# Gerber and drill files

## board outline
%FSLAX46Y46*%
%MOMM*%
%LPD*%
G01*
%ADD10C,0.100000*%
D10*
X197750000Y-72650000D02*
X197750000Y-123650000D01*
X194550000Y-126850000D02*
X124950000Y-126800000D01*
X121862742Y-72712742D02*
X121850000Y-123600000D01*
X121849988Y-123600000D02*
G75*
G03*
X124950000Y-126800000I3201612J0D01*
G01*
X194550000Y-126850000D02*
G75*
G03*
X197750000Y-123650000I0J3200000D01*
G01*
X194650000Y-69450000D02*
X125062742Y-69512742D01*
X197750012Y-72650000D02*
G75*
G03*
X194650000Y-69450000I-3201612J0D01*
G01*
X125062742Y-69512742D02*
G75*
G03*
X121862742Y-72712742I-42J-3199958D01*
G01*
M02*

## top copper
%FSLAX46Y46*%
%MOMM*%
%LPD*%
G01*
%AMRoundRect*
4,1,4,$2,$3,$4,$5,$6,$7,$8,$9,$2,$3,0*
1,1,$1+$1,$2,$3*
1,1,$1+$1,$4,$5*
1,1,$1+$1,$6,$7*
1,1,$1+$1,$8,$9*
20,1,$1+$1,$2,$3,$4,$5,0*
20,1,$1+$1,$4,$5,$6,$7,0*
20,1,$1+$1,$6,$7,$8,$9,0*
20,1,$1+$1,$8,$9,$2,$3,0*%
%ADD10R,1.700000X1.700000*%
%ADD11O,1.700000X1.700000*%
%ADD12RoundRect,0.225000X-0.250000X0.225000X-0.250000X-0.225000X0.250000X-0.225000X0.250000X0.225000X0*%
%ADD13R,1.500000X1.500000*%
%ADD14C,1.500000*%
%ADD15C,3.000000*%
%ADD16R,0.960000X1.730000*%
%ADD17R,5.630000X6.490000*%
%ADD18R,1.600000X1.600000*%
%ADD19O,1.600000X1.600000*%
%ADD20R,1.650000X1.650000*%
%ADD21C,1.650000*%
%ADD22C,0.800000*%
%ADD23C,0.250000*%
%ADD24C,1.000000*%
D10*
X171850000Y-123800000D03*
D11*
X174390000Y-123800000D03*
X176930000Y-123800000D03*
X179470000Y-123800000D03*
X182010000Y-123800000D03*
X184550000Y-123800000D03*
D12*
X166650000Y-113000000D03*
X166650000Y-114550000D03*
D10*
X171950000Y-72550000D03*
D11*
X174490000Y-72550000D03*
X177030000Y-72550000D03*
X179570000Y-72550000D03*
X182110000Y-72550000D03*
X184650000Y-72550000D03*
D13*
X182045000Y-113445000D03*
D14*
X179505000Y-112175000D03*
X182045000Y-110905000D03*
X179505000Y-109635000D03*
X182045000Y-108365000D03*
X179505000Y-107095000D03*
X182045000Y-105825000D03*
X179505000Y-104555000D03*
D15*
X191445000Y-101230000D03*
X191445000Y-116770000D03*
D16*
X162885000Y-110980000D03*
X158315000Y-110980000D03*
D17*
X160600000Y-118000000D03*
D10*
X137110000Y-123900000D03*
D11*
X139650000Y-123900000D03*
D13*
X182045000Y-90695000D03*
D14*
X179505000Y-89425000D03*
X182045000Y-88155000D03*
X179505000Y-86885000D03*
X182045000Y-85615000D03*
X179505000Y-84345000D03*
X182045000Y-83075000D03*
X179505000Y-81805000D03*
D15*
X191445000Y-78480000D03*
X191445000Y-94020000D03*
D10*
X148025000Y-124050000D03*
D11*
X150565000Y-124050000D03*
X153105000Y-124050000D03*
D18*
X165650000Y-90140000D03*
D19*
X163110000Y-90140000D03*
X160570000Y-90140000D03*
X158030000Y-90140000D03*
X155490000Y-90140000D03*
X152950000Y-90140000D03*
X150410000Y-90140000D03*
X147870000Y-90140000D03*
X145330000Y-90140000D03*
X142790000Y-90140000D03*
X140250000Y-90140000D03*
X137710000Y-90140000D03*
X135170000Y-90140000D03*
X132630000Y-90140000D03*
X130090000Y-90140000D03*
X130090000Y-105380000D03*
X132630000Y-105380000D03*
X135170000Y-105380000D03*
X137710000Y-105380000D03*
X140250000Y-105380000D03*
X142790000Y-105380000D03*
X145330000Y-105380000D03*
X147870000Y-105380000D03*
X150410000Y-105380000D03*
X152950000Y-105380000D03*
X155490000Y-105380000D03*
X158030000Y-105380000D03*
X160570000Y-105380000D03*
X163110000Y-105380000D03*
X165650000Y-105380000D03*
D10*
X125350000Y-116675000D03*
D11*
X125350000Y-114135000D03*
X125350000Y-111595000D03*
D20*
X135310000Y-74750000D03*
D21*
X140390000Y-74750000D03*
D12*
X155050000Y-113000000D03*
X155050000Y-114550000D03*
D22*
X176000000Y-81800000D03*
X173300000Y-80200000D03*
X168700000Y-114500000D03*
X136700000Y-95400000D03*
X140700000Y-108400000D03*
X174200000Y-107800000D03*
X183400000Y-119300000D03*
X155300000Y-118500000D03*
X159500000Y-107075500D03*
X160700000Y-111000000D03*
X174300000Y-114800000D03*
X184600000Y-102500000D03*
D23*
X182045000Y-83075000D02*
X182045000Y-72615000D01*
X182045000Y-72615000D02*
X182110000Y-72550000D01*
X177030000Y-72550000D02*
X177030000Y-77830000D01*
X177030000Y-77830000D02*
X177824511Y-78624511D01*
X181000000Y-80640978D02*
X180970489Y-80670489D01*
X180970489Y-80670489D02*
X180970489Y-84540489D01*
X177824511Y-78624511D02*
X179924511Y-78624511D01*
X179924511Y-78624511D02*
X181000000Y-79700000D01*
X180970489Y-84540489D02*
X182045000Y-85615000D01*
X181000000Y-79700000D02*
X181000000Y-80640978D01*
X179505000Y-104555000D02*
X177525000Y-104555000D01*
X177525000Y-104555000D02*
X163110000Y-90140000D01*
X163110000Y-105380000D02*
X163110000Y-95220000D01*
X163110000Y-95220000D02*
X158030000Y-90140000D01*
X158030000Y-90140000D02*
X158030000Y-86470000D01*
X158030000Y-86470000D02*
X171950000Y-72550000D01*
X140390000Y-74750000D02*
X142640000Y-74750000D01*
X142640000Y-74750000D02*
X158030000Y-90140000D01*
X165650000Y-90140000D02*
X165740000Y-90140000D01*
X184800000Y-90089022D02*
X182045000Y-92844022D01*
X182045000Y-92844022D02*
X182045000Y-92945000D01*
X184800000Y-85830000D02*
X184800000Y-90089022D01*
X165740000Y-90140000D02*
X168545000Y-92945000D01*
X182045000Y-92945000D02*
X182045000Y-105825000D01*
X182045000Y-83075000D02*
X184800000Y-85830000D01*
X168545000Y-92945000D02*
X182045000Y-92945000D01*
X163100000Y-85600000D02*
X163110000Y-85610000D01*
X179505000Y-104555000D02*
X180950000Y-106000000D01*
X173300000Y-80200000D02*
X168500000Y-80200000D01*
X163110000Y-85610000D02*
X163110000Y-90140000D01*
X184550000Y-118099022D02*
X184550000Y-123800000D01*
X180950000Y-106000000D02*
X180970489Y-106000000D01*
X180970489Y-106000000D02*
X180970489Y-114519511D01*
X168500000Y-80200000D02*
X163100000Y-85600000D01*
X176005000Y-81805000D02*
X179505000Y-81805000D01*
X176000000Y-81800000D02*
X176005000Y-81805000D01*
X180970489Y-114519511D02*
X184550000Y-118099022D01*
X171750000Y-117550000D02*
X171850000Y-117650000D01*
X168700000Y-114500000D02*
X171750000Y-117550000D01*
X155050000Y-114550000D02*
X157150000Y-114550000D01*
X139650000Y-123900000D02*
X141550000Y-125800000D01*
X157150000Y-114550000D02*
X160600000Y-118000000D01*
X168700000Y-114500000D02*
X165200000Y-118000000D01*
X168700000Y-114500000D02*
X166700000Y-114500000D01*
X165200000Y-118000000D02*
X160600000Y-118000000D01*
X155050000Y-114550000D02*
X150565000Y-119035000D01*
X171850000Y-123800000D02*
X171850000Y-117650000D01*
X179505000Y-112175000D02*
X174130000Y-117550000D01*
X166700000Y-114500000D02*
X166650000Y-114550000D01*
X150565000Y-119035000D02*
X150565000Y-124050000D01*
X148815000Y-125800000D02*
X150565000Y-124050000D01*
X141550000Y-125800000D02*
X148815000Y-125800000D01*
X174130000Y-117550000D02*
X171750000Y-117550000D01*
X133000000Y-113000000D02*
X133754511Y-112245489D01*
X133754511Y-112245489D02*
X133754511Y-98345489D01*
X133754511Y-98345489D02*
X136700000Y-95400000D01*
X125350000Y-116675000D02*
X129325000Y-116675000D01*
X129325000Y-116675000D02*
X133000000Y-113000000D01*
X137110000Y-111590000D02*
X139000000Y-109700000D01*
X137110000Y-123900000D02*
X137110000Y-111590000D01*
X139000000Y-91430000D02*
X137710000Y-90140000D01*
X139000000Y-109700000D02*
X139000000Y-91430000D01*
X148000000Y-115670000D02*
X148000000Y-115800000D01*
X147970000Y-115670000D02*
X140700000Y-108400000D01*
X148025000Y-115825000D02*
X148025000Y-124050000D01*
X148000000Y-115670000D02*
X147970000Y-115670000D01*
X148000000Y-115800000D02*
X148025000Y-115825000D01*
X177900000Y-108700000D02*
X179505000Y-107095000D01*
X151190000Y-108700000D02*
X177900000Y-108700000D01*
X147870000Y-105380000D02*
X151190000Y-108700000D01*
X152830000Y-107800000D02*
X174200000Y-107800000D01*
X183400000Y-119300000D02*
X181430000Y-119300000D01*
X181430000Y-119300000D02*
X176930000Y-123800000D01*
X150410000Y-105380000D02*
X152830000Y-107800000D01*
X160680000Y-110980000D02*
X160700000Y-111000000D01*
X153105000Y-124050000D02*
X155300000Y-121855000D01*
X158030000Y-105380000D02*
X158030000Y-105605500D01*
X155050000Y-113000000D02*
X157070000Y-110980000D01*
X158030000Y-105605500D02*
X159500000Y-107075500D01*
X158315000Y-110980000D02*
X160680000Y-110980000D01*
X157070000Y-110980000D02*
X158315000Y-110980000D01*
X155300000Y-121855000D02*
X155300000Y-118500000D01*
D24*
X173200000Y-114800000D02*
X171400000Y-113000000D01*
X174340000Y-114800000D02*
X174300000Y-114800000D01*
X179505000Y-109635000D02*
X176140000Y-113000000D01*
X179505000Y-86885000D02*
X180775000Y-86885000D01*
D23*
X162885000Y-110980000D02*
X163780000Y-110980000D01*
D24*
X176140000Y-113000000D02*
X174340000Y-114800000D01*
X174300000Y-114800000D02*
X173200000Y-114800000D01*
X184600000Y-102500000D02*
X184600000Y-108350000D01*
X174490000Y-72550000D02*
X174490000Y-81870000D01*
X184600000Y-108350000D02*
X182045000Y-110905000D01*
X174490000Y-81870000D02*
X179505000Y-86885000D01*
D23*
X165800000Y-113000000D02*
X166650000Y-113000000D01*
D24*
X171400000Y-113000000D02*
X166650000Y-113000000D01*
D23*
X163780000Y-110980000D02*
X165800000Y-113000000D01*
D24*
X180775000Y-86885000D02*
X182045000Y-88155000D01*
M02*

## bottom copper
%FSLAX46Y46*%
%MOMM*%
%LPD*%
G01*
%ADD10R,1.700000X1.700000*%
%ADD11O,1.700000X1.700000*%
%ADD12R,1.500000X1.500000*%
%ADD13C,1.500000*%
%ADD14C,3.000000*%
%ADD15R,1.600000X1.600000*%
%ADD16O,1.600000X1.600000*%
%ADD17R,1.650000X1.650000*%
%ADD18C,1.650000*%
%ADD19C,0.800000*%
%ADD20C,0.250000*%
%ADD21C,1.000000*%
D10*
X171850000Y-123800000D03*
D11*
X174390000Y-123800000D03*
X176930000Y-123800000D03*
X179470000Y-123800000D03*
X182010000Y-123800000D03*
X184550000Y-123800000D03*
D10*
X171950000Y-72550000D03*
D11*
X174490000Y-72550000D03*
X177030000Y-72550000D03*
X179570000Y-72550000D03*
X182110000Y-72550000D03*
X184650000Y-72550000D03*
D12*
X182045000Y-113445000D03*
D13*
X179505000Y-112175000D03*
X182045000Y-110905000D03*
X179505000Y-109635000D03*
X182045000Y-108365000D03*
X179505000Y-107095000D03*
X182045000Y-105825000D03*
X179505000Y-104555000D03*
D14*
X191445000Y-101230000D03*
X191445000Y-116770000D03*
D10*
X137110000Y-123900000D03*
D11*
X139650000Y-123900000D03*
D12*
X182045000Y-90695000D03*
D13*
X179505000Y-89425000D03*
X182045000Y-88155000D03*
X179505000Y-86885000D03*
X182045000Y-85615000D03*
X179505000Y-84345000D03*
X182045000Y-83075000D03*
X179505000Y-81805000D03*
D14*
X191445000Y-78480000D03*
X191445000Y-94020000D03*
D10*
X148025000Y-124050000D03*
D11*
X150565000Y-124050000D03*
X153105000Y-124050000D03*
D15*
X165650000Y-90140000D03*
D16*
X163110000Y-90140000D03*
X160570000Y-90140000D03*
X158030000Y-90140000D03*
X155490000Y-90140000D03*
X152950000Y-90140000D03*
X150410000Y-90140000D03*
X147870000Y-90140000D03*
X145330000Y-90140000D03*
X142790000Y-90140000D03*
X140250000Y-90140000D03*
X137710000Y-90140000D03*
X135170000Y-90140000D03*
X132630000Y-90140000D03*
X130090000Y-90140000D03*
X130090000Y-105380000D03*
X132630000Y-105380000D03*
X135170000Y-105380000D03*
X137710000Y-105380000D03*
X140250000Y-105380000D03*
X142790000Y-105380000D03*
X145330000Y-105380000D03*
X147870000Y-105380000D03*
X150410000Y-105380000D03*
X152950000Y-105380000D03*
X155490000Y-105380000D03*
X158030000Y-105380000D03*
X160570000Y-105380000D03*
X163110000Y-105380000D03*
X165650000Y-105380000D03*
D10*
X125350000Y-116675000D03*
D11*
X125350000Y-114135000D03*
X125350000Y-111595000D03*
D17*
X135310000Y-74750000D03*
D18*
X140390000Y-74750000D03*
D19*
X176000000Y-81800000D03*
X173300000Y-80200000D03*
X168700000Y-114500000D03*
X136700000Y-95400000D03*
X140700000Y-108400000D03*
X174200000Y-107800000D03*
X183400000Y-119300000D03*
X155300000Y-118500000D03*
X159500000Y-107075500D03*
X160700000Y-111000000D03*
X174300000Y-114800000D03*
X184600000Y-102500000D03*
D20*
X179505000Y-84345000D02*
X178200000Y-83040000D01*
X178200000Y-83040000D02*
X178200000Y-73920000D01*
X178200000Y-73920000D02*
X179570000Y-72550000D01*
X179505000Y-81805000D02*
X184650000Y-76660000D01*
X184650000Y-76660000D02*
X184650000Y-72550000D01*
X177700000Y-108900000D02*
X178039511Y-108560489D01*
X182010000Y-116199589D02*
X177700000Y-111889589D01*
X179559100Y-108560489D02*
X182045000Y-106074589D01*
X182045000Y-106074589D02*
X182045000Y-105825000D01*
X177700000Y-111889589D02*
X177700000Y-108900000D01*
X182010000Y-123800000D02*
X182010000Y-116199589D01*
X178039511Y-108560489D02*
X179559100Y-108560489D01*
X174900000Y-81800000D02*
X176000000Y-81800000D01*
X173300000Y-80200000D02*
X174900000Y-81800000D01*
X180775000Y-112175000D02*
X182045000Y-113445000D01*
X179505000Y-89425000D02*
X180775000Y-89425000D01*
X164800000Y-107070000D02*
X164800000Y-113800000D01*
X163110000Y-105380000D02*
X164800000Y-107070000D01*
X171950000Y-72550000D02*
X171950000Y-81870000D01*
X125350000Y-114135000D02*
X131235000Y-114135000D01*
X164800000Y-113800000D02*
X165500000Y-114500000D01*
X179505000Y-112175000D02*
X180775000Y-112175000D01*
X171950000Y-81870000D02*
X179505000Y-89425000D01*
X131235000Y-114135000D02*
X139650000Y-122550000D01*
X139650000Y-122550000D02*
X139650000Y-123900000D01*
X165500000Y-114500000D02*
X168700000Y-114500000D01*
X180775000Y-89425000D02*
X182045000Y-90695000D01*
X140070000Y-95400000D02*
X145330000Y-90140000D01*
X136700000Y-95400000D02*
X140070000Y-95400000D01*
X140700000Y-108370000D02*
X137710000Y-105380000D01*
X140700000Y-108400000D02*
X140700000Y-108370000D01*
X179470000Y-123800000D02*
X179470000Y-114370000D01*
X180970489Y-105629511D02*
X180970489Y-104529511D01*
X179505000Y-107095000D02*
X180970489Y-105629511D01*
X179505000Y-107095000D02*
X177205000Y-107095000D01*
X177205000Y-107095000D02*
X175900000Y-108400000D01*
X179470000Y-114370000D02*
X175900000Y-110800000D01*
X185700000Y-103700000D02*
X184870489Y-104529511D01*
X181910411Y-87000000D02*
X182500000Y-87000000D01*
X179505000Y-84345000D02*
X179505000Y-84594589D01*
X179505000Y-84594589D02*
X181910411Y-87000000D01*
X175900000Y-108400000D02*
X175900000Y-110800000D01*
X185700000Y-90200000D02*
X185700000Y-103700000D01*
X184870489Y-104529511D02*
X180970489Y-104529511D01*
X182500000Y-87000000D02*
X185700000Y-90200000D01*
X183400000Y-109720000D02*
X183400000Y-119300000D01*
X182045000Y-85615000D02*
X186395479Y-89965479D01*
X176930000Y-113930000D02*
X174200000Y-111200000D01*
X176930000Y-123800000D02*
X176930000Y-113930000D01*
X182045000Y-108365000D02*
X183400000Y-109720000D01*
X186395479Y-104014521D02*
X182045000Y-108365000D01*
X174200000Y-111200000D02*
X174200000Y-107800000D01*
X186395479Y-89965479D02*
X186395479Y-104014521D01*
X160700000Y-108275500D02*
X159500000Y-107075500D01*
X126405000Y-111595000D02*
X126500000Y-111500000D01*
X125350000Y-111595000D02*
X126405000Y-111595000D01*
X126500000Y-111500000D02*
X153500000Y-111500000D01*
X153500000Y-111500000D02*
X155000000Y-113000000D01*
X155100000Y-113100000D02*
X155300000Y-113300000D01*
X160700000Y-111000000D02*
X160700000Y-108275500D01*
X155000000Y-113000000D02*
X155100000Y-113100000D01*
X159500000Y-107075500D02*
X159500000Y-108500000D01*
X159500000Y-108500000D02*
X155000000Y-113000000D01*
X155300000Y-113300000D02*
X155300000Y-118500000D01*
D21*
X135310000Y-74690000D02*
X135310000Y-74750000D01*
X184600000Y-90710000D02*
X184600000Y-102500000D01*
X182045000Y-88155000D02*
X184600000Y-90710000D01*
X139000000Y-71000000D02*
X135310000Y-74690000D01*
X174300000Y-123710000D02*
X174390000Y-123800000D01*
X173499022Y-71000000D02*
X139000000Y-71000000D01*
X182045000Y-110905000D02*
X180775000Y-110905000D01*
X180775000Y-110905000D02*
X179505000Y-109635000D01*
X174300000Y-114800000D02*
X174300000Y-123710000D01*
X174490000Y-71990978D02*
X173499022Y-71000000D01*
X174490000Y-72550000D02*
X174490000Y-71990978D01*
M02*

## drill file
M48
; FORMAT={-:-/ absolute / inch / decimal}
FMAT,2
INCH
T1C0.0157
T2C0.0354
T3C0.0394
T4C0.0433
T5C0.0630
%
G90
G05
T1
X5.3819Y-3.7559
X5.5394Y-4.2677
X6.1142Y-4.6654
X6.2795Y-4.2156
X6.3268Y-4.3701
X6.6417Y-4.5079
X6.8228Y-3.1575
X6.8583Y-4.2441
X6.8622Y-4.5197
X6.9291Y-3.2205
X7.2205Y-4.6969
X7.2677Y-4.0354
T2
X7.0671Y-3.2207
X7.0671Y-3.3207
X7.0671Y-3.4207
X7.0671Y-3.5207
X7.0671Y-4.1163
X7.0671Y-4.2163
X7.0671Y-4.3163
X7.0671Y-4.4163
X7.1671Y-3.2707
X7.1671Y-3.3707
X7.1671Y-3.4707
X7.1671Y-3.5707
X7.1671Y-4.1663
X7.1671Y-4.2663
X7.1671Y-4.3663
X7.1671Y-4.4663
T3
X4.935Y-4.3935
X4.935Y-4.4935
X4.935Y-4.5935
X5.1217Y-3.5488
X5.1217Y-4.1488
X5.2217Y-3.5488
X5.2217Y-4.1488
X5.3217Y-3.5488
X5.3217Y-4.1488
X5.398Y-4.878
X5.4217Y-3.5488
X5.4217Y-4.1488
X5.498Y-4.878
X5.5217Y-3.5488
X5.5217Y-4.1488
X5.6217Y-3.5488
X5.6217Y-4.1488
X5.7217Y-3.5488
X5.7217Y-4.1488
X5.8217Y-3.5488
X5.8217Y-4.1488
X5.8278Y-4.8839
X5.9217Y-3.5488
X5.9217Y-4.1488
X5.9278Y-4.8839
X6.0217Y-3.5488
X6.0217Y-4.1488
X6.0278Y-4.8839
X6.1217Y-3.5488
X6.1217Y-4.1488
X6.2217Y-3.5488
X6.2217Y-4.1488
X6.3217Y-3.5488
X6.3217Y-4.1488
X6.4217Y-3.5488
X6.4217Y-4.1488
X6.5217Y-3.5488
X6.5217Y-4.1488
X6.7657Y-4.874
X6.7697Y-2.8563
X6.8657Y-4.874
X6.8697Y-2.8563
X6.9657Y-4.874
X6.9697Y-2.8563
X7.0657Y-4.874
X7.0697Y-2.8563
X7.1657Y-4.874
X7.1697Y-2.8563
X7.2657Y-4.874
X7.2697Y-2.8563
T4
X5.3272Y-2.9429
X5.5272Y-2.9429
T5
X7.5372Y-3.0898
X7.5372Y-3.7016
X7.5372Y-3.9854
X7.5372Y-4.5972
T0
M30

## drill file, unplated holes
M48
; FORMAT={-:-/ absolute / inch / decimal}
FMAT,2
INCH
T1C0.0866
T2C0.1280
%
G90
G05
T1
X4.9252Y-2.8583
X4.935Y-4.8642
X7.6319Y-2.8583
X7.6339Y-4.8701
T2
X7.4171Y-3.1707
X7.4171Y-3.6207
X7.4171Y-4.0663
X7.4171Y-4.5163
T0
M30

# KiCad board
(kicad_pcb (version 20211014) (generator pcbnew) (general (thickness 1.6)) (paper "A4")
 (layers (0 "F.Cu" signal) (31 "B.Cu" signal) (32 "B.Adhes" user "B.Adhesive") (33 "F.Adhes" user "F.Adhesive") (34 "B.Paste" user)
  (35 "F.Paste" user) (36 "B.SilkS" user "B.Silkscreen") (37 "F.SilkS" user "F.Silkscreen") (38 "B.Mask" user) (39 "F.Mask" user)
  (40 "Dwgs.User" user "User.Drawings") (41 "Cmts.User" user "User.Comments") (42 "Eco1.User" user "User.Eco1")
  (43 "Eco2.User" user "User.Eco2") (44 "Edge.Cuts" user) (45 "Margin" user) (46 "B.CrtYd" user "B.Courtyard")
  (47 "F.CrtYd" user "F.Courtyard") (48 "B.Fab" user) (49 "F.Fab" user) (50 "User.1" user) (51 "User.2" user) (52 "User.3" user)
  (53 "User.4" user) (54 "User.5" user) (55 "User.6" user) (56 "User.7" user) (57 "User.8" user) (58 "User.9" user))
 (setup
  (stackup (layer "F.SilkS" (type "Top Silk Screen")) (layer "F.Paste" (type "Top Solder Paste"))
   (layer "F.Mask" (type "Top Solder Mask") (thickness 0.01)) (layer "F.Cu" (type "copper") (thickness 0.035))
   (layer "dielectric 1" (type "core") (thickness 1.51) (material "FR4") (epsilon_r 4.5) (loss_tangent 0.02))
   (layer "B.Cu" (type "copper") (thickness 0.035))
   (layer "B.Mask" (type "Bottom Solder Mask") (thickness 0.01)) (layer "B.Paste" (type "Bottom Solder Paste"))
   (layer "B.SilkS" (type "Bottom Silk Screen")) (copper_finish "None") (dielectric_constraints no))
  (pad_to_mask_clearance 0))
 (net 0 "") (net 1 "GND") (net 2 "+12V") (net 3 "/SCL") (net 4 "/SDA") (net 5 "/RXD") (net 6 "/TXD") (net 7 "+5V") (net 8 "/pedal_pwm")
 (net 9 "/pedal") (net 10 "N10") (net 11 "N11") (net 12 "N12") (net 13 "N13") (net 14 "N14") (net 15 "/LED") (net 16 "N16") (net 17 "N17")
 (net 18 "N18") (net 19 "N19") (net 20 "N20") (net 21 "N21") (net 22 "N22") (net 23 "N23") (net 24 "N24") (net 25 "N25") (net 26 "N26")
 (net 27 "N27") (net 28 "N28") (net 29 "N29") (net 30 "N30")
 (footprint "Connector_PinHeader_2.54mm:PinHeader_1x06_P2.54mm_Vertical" (layer "F.Cu") (at 171.85 123.8 90)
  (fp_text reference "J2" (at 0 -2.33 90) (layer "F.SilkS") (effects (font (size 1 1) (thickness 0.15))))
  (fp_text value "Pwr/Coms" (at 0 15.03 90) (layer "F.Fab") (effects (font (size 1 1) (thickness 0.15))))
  (pad "1" thru_hole rect (at 0 0 90) (size 1.7 1.7) (drill 1) (layers *.Cu *.Mask) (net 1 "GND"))
  (pad "2" thru_hole oval (at 0 2.54 90) (size 1.7 1.7) (drill 1) (layers *.Cu *.Mask) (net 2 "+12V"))
  (pad "3" thru_hole oval (at 0 5.08 90) (size 1.7 1.7) (drill 1) (layers *.Cu *.Mask) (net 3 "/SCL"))
  (pad "4" thru_hole oval (at 0 7.62 90) (size 1.7 1.7) (drill 1) (layers *.Cu *.Mask) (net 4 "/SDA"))
  (pad "5" thru_hole oval (at 0 10.16 90) (size 1.7 1.7) (drill 1) (layers *.Cu *.Mask) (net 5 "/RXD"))
  (pad "6" thru_hole oval (at 0 12.7 90) (size 1.7 1.7) (drill 1) (layers *.Cu *.Mask) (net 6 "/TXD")))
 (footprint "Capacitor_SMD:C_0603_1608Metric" (layer "F.Cu") (at 166.65 113.775 -90)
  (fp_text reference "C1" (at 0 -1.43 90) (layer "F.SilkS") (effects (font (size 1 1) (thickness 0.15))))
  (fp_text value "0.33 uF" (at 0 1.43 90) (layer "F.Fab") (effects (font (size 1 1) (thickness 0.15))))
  (pad "1" smd roundrect (at -0.775 0 270) (size 0.9 0.95) (layers "F.Cu" "F.Paste" "F.Mask") (roundrect_rratio 0.25) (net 2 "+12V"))
  (pad "2" smd roundrect (at 0.775 0 270) (size 0.9 0.95) (layers "F.Cu" "F.Paste" "F.Mask") (roundrect_rratio 0.25) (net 1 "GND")))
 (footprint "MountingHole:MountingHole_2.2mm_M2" (layer "F.Cu") (at 193.9 123.7)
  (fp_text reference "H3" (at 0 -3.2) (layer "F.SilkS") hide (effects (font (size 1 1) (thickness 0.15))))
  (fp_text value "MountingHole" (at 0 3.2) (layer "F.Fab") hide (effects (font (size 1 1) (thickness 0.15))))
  (pad "" np_thru_hole circle (at 0 0) (size 2.2 2.2) (drill 2.2) (layers *.Cu *.Mask)))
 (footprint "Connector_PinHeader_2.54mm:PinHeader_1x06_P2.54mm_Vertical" (layer "F.Cu") (at 171.95 72.55 90)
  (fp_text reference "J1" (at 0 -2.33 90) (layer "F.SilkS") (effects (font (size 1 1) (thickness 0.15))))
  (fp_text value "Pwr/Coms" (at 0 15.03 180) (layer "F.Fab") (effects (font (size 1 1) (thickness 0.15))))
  (pad "1" thru_hole rect (at 0 0 90) (size 1.7 1.7) (drill 1) (layers *.Cu *.Mask) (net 1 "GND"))
  (pad "2" thru_hole oval (at 0 2.54 90) (size 1.7 1.7) (drill 1) (layers *.Cu *.Mask) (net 2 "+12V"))
  (pad "3" thru_hole oval (at 0 5.08 90) (size 1.7 1.7) (drill 1) (layers *.Cu *.Mask) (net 3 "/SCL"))
  (pad "4" thru_hole oval (at 0 7.62 90) (size 1.7 1.7) (drill 1) (layers *.Cu *.Mask) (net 4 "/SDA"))
  (pad "5" thru_hole oval (at 0 10.16 90) (size 1.7 1.7) (drill 1) (layers *.Cu *.Mask) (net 5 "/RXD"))
  (pad "6" thru_hole oval (at 0 12.7 90) (size 1.7 1.7) (drill 1) (layers *.Cu *.Mask) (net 6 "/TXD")))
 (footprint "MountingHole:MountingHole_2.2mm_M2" (layer "F.Cu") (at 125.1 72.6)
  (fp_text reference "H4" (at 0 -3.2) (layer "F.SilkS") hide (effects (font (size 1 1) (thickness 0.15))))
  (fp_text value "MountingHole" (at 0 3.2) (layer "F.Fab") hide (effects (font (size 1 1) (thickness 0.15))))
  (pad "" np_thru_hole circle (at 0 0) (size 2.2 2.2) (drill 2.2) (layers *.Cu *.Mask)))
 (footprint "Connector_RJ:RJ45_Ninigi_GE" (layer "F.Cu") (at 182.045 113.445 90)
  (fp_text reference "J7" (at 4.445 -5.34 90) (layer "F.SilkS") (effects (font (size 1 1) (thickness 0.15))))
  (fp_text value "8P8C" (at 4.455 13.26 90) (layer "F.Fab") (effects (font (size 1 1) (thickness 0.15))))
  (pad "" np_thru_hole circle (at 10.16 6.35 270) (size 3.25 3.25) (drill 3.25) (layers *.Cu *.Mask))
  (pad "" np_thru_hole circle (at -1.27 6.35 90) (size 3.25 3.25) (drill 3.25) (layers *.Cu *.Mask))
  (pad "1" thru_hole rect (at 0 0 270) (size 1.5 1.5) (drill 0.9) (layers *.Cu *.Mask) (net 1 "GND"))
  (pad "2" thru_hole circle (at 1.27 -2.54 270) (size 1.5 1.5) (drill 0.9) (layers *.Cu *.Mask) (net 1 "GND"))
  (pad "3" thru_hole circle (at 2.54 0 270) (size 1.5 1.5) (drill 0.9) (layers *.Cu *.Mask) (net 2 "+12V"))
  (pad "4" thru_hole circle (at 3.81 -2.54 270) (size 1.5 1.5) (drill 0.9) (layers *.Cu *.Mask) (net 2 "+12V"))
  (pad "5" thru_hole circle (at 5.08 0 270) (size 1.5 1.5) (drill 0.9) (layers *.Cu *.Mask) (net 3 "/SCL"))
  (pad "6" thru_hole circle (at 6.35 -2.54 270) (size 1.5 1.5) (drill 0.9) (layers *.Cu *.Mask) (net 4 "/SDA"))
  (pad "7" thru_hole circle (at 7.62 0 270) (size 1.5 1.5) (drill 0.9) (layers *.Cu *.Mask) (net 5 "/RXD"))
  (pad "8" thru_hole circle (at 8.89 -2.54 270) (size 1.5 1.5) (drill 0.9) (layers *.Cu *.Mask) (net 6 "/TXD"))
  (pad "SH" thru_hole circle (at 12.215 9.4 270) (size 3 3) (drill 1.6) (layers *.Cu *.Mask))
  (pad "SH" thru_hole circle (at -3.325 9.4 90) (size 3 3) (drill 1.6) (layers *.Cu *.Mask)))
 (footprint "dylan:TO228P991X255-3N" (layer "F.Cu") (at 160.6 115.68 -90)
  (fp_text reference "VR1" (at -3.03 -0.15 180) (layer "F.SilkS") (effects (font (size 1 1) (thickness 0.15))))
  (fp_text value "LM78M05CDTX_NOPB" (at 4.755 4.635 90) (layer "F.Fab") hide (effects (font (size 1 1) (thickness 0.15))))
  (pad "1" smd rect locked (at -4.7 -2.285 270) (size 1.73 0.96) (layers "F.Cu" "F.Paste" "F.Mask") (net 2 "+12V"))
  (pad "3" smd rect locked (at -4.7 2.285 270) (size 1.73 0.96) (layers "F.Cu" "F.Paste" "F.Mask") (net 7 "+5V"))
  (pad "4" smd rect locked (at 2.32 0 270) (size 6.49 5.63) (layers "F.Cu" "F.Mask") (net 1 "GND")))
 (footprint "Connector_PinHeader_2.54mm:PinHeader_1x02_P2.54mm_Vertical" (layer "F.Cu") (at 137.11 123.9 90)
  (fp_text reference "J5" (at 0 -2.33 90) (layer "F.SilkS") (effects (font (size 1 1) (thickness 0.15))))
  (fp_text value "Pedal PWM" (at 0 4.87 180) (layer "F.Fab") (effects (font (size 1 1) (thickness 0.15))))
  (pad "1" thru_hole rect (at 0 0 90) (size 1.7 1.7) (drill 1) (layers *.Cu *.Mask) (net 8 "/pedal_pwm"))
  (pad "2" thru_hole oval (at 0 2.54 90) (size 1.7 1.7) (drill 1) (layers *.Cu *.Mask) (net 1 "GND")))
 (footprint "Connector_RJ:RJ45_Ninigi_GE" (layer "F.Cu") (at 182.045 90.695 90)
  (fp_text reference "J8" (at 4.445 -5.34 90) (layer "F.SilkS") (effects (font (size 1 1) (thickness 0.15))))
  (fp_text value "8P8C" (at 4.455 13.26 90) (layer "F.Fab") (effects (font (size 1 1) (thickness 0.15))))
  (pad "" np_thru_hole circle (at 10.16 6.35 270) (size 3.25 3.25) (drill 3.25) (layers *.Cu *.Mask))
  (pad "" np_thru_hole circle (at -1.27 6.35 90) (size 3.25 3.25) (drill 3.25) (layers *.Cu *.Mask))
  (pad "1" thru_hole rect (at 0 0 270) (size 1.5 1.5) (drill 0.9) (layers *.Cu *.Mask) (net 1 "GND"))
  (pad "2" thru_hole circle (at 1.27 -2.54 270) (size 1.5 1.5) (drill 0.9) (layers *.Cu *.Mask) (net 1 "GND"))
  (pad "3" thru_hole circle (at 2.54 0 270) (size 1.5 1.5) (drill 0.9) (layers *.Cu *.Mask) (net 2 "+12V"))
  (pad "4" thru_hole circle (at 3.81 -2.54 270) (size 1.5 1.5) (drill 0.9) (layers *.Cu *.Mask) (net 2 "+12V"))
  (pad "5" thru_hole circle (at 5.08 0 270) (size 1.5 1.5) (drill 0.9) (layers *.Cu *.Mask) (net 3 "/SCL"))
  (pad "6" thru_hole circle (at 6.35 -2.54 270) (size 1.5 1.5) (drill 0.9) (layers *.Cu *.Mask) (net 4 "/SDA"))
  (pad "7" thru_hole circle (at 7.62 0 270) (size 1.5 1.5) (drill 0.9) (layers *.Cu *.Mask) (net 5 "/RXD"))
  (pad "8" thru_hole circle (at 8.89 -2.54 270) (size 1.5 1.5) (drill 0.9) (layers *.Cu *.Mask) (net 6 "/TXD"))
  (pad "SH" thru_hole circle (at 12.215 9.4 270) (size 3 3) (drill 1.6) (layers *.Cu *.Mask))
  (pad "SH" thru_hole circle (at -3.325 9.4 90) (size 3 3) (drill 1.6) (layers *.Cu *.Mask)))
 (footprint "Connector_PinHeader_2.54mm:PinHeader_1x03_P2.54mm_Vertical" (layer "F.Cu") (at 148.025 124.05 90)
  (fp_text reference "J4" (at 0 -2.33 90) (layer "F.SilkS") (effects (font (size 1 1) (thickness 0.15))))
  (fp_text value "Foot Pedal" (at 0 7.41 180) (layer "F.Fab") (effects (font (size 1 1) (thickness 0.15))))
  (pad "1" thru_hole rect (at 0 0 90) (size 1.7 1.7) (drill 1) (layers *.Cu *.Mask) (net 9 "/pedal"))
  (pad "2" thru_hole oval (at 0 2.54 90) (size 1.7 1.7) (drill 1) (layers *.Cu *.Mask) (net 1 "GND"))
  (pad "3" thru_hole oval (at 0 5.08 90) (size 1.7 1.7) (drill 1) (layers *.Cu *.Mask) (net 7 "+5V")))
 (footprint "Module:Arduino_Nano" (layer "F.Cu") (at 165.65 90.14 -90)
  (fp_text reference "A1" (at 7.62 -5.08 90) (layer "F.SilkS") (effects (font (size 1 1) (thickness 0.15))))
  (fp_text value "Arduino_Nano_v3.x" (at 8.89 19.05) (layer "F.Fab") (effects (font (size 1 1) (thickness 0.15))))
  (pad "1" thru_hole rect (at 0 0 270) (size 1.6 1.6) (drill 1) (layers *.Cu *.Mask) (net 5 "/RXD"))
  (pad "2" thru_hole oval (at 0 2.54 270) (size 1.6 1.6) (drill 1) (layers *.Cu *.Mask) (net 6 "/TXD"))
  (pad "3" thru_hole oval (at 0 5.08 270) (size 1.6 1.6) (drill 1) (layers *.Cu *.Mask) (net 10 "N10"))
  (pad "4" thru_hole oval (at 0 7.62 270) (size 1.6 1.6) (drill 1) (layers *.Cu *.Mask) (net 1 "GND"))
  (pad "5" thru_hole oval (at 0 10.16 270) (size 1.6 1.6) (drill 1) (layers *.Cu *.Mask) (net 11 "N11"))
  (pad "6" thru_hole oval (at 0 12.7 270) (size 1.6 1.6) (drill 1) (layers *.Cu *.Mask) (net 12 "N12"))
  (pad "7" thru_hole oval (at 0 15.24 270) (size 1.6 1.6) (drill 1) (layers *.Cu *.Mask) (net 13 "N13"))
  (pad "8" thru_hole oval (at 0 17.78 270) (size 1.6 1.6) (drill 1) (layers *.Cu *.Mask) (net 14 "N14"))
  (pad "9" thru_hole oval (at 0 20.32 270) (size 1.6 1.6) (drill 1) (layers *.Cu *.Mask) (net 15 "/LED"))
  (pad "10" thru_hole oval (at 0 22.86 270) (size 1.6 1.6) (drill 1) (layers *.Cu *.Mask) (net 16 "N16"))
  (pad "11" thru_hole oval (at 0 25.4 270) (size 1.6 1.6) (drill 1) (layers *.Cu *.Mask) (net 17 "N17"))
  (pad "12" thru_hole oval (at 0 27.94 270) (size 1.6 1.6) (drill 1) (layers *.Cu *.Mask) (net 8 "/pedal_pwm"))
  (pad "13" thru_hole oval (at 0 30.48 270) (size 1.6 1.6) (drill 1) (layers *.Cu *.Mask) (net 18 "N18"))
  (pad "14" thru_hole oval (at 0 33.02 270) (size 1.6 1.6) (drill 1) (layers *.Cu *.Mask) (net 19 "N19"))
  (pad "15" thru_hole oval (at 0 35.56 270) (size 1.6 1.6) (drill 1) (layers *.Cu *.Mask) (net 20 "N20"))
  (pad "16" thru_hole oval (at 15.24 35.56 270) (size 1.6 1.6) (drill 1) (layers *.Cu *.Mask) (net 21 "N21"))
  (pad "17" thru_hole oval (at 15.24 33.02 270) (size 1.6 1.6) (drill 1) (layers *.Cu *.Mask) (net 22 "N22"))
  (pad "18" thru_hole oval (at 15.24 30.48 270) (size 1.6 1.6) (drill 1) (layers *.Cu *.Mask) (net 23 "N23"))
  (pad "19" thru_hole oval (at 15.24 27.94 270) (size 1.6 1.6) (drill 1) (layers *.Cu *.Mask) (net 9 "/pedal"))
  (pad "20" thru_hole oval (at 15.24 25.4 270) (size 1.6 1.6) (drill 1) (layers *.Cu *.Mask) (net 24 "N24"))
  (pad "21" thru_hole oval (at 15.24 22.86 270) (size 1.6 1.6) (drill 1) (layers *.Cu *.Mask) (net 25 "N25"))
  (pad "22" thru_hole oval (at 15.24 20.32 270) (size 1.6 1.6) (drill 1) (layers *.Cu *.Mask) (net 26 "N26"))
  (pad "23" thru_hole oval (at 15.24 17.78 270) (size 1.6 1.6) (drill 1) (layers *.Cu *.Mask) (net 4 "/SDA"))
  (pad "24" thru_hole oval (at 15.24 15.24 270) (size 1.6 1.6) (drill 1) (layers *.Cu *.Mask) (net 3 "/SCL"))
  (pad "25" thru_hole oval (at 15.24 12.7 270) (size 1.6 1.6) (drill 1) (layers *.Cu *.Mask) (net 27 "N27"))
  (pad "26" thru_hole oval (at 15.24 10.16 270) (size 1.6 1.6) (drill 1) (layers *.Cu *.Mask) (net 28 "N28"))
  (pad "27" thru_hole oval (at 15.24 7.62 270) (size 1.6 1.6) (drill 1) (layers *.Cu *.Mask) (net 7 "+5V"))
  (pad "28" thru_hole oval (at 15.24 5.08 270) (size 1.6 1.6) (drill 1) (layers *.Cu *.Mask) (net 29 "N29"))
  (pad "29" thru_hole oval (at 15.24 2.54 270) (size 1.6 1.6) (drill 1) (layers *.Cu *.Mask) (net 1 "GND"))
  (pad "30" thru_hole oval (at 15.24 0 270) (size 1.6 1.6) (drill 1) (layers *.Cu *.Mask) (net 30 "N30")))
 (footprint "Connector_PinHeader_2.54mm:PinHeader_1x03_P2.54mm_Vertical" (layer "F.Cu") (at 125.35 116.675 180)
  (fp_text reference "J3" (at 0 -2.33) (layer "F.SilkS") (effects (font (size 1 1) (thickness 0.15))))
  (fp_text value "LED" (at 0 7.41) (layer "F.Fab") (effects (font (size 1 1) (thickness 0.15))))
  (pad "1" thru_hole rect (at 0 0 180) (size 1.7 1.7) (drill 1) (layers *.Cu *.Mask) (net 15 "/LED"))
  (pad "2" thru_hole oval (at 0 2.54 180) (size 1.7 1.7) (drill 1) (layers *.Cu *.Mask) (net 1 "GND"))
  (pad "3" thru_hole oval (at 0 5.08 180) (size 1.7 1.7) (drill 1) (layers *.Cu *.Mask) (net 7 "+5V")))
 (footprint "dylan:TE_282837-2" (layer "F.Cu") (at 137.85 74.75)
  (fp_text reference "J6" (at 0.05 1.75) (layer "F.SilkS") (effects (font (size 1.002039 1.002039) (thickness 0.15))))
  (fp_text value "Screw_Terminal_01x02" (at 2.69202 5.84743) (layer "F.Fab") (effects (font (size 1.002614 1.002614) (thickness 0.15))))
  (pad "1" thru_hole rect locked (at -2.54 0) (size 1.65 1.65) (drill 1.1) (layers *.Cu *.Mask) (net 2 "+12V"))
  (pad "2" thru_hole circle locked (at 2.54 0) (size 1.65 1.65) (drill 1.1) (layers *.Cu *.Mask) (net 1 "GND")))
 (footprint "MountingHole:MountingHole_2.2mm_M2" (layer "F.Cu") (at 193.85 72.6)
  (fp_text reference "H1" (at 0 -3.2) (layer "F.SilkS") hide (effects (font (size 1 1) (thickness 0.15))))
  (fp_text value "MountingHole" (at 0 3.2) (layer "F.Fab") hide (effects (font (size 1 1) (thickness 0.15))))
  (pad "" np_thru_hole circle (at 0 0) (size 2.2 2.2) (drill 2.2) (layers *.Cu *.Mask)))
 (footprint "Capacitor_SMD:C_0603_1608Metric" (layer "F.Cu") (at 155.05 113.775 -90)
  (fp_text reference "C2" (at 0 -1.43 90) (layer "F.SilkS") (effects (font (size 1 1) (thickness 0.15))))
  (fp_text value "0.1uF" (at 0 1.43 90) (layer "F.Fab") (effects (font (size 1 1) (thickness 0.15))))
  (pad "1" smd roundrect (at -0.775 0 270) (size 0.9 0.95) (layers "F.Cu" "F.Paste" "F.Mask") (roundrect_rratio 0.25) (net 7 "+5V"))
  (pad "2" smd roundrect (at 0.775 0 270) (size 0.9 0.95) (layers "F.Cu" "F.Paste" "F.Mask") (roundrect_rratio 0.25) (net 1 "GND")))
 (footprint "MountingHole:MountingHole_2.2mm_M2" (layer "F.Cu") (at 125.35 123.55)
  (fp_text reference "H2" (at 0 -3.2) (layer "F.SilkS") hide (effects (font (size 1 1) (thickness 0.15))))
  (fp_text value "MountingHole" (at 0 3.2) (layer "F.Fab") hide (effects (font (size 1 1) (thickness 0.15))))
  (pad "" np_thru_hole circle (at 0 0) (size 2.2 2.2) (drill 2.2) (layers *.Cu *.Mask)))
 (gr_line (start 197.75 72.65) (end 197.75 123.65) (layer "Edge.Cuts") (width 0.1))
 (gr_line (start 194.55 126.85) (end 124.95 126.8) (layer "Edge.Cuts") (width 0.1))
 (gr_line (start 121.862742 72.712742) (end 121.85 123.6) (layer "Edge.Cuts") (width 0.1))
 (gr_arc (start 124.95 126.8) (mid 122.752085 125.827667) (end 121.85 123.6) (layer "Edge.Cuts") (width 0.1))
 (gr_arc (start 197.75 123.65) (mid 196.812742 125.912742) (end 194.55 126.85) (layer "Edge.Cuts") (width 0.1))
 (gr_line (start 194.65 69.45) (end 125.062742 69.512742) (layer "Edge.Cuts") (width 0.1))
 (gr_arc (start 194.65 69.45) (mid 196.847914 70.422333) (end 197.75 72.65) (layer "Edge.Cuts") (width 0.1))
 (gr_arc (start 121.862742 72.712742) (mid 122.8 70.45) (end 125.062742 69.512742) (layer "Edge.Cuts") (width 0.1))
 (segment (start 165.65 90.14) (end 165.74 90.14) (width 0.25) (layer "F.Cu") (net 5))
 (segment (start 182.045 72.615) (end 182.11 72.55) (width 0.25) (layer "F.Cu") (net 5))
 (segment (start 184.8 90.089022) (end 182.045 92.844022) (width 0.25) (layer "F.Cu") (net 5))
 (segment (start 182.045 92.844022) (end 182.045 92.945) (width 0.25) (layer "F.Cu") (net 5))
 (segment (start 184.8 85.83) (end 184.8 90.089022) (width 0.25) (layer "F.Cu") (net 5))
 (segment (start 165.74 90.14) (end 168.545 92.945) (width 0.25) (layer "F.Cu") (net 5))
 (segment (start 182.045 92.945) (end 182.045 105.825) (width 0.25) (layer "F.Cu") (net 5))
 (segment (start 182.045 83.075) (end 184.8 85.83) (width 0.25) (layer "F.Cu") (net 5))
 (segment (start 168.545 92.945) (end 182.045 92.945) (width 0.25) (layer "F.Cu") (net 5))
 (segment (start 182.045 83.075) (end 182.045 72.615) (width 0.25) (layer "F.Cu") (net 5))
 (segment (start 177.7 108.9) (end 178.039511 108.560489) (width 0.25) (layer "B.Cu") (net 5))
 (segment (start 182.01 116.199589) (end 177.7 111.889589) (width 0.25) (layer "B.Cu") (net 5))
 (segment (start 179.5591 108.560489) (end 182.045 106.074589) (width 0.25) (layer "B.Cu") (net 5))
 (segment (start 182.045 106.074589) (end 182.045 105.825) (width 0.25) (layer "B.Cu") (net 5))
 (segment (start 177.7 111.889589) (end 177.7 108.9) (width 0.25) (layer "B.Cu") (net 5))
 (segment (start 182.01 123.8) (end 182.01 116.199589) (width 0.25) (layer "B.Cu") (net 5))
 (segment (start 178.039511 108.560489) (end 179.5591 108.560489) (width 0.25) (layer "B.Cu") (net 5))
 (segment (start 163.1 85.6) (end 163.11 85.61) (width 0.25) (layer "F.Cu") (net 6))
 (segment (start 179.505 104.555) (end 180.95 106) (width 0.25) (layer "F.Cu") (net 6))
 (segment (start 177.525 104.555) (end 163.11 90.14) (width 0.25) (layer "F.Cu") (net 6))
 (segment (start 173.3 80.2) (end 168.5 80.2) (width 0.25) (layer "F.Cu") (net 6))
 (segment (start 163.11 85.61) (end 163.11 90.14) (width 0.25) (layer "F.Cu") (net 6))
 (segment (start 184.55 118.099022) (end 184.55 123.8) (width 0.25) (layer "F.Cu") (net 6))
 (segment (start 180.95 106) (end 180.970489 106) (width 0.25) (layer "F.Cu") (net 6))
 (segment (start 179.505 104.555) (end 177.525 104.555) (width 0.25) (layer "F.Cu") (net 6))
 (segment (start 180.970489 106) (end 180.970489 114.519511) (width 0.25) (layer "F.Cu") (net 6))
 (segment (start 168.5 80.2) (end 163.1 85.6) (width 0.25) (layer "F.Cu") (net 6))
 (segment (start 176.005 81.805) (end 179.505 81.805) (width 0.25) (layer "F.Cu") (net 6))
 (segment (start 176 81.8) (end 176.005 81.805) (width 0.25) (layer "F.Cu") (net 6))
 (segment (start 180.970489 114.519511) (end 184.55 118.099022) (width 0.25) (layer "F.Cu") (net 6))
 (via (at 176 81.8) (size 0.8) (drill 0.4) (layers "F.Cu" "B.Cu") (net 6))
 (via (at 173.3 80.2) (size 0.8) (drill 0.4) (layers "F.Cu" "B.Cu") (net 6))
 (segment (start 174.9 81.8) (end 176 81.8) (width 0.25) (layer "B.Cu") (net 6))
 (segment (start 179.505 81.805) (end 184.65 76.66) (width 0.25) (layer "B.Cu") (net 6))
 (segment (start 184.65 76.66) (end 184.65 72.55) (width 0.25) (layer "B.Cu") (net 6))
 (segment (start 173.3 80.2) (end 174.9 81.8) (width 0.25) (layer "B.Cu") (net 6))
 (segment (start 171.75 117.55) (end 171.85 117.65) (width 0.25) (layer "F.Cu") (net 1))
 (segment (start 168.7 114.5) (end 171.75 117.55) (width 0.25) (layer "F.Cu") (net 1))
 (segment (start 163.11 95.22) (end 158.03 90.14) (width 0.25) (layer "F.Cu") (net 1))
 (segment (start 155.05 114.55) (end 157.15 114.55) (width 0.25) (layer "F.Cu") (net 1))
 (segment (start 139.65 123.9) (end 141.55 125.8) (width 0.25) (layer "F.Cu") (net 1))
 (segment (start 140.39 74.75) (end 142.64 74.75) (width 0.25) (layer "F.Cu") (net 1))
 (segment (start 157.15 114.55) (end 160.6 118) (width 0.25) (layer "F.Cu") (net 1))
 (segment (start 142.64 74.75) (end 158.03 90.14) (width 0.25) (layer "F.Cu") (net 1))
 (segment (start 168.7 114.5) (end 165.2 118) (width 0.25) (layer "F.Cu") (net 1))
 (segment (start 158.03 86.47) (end 171.95 72.55) (width 0.25) (layer "F.Cu") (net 1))
 (segment (start 168.7 114.5) (end 166.7 114.5) (width 0.25) (layer "F.Cu") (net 1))
 (segment (start 165.2 118) (end 160.6 118) (width 0.25) (layer "F.Cu") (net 1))
 (segment (start 155.05 114.55) (end 150.565 119.035) (width 0.25) (layer "F.Cu") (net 1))
 (segment (start 171.85 123.8) (end 171.85 117.65) (width 0.25) (layer "F.Cu") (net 1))
 (segment (start 179.505 112.175) (end 174.13 117.55) (width 0.25) (layer "F.Cu") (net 1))
 (segment (start 158.03 90.14) (end 158.03 86.47) (width 0.25) (layer "F.Cu") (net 1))
 (segment (start 166.7 114.5) (end 166.65 114.55) (width 0.25) (layer "F.Cu") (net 1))
 (segment (start 163.11 105.38) (end 163.11 95.22) (width 0.25) (layer "F.Cu") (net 1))
 (segment (start 150.565 119.035) (end 150.565 124.05) (width 0.25) (layer "F.Cu") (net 1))
 (segment (start 148.815 125.8) (end 150.565 124.05) (width 0.25) (layer "F.Cu") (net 1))
 (segment (start 141.55 125.8) (end 148.815 125.8) (width 0.25) (layer "F.Cu") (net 1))
 (segment (start 174.13 117.55) (end 171.75 117.55) (width 0.25) (layer "F.Cu") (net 1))
 (via (at 168.7 114.5) (size 0.8) (drill 0.4) (layers "F.Cu" "B.Cu") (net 1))
 (segment (start 180.775 112.175) (end 182.045 113.445) (width 0.25) (layer "B.Cu") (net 1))
 (segment (start 179.505 89.425) (end 180.775 89.425) (width 0.25) (layer "B.Cu") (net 1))
 (segment (start 164.8 107.07) (end 164.8 113.8) (width 0.25) (layer "B.Cu") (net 1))
 (segment (start 163.11 105.38) (end 164.8 107.07) (width 0.25) (layer "B.Cu") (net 1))
 (segment (start 171.95 72.55) (end 171.95 81.87) (width 0.25) (layer "B.Cu") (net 1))
 (segment (start 125.35 114.135) (end 131.235 114.135) (width 0.25) (layer "B.Cu") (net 1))
 (segment (start 164.8 113.8) (end 165.5 114.5) (width 0.25) (layer "B.Cu") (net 1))
 (segment (start 179.505 112.175) (end 180.775 112.175) (width 0.25) (layer "B.Cu") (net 1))
 (segment (start 171.95 81.87) (end 179.505 89.425) (width 0.25) (layer "B.Cu") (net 1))
 (segment (start 131.235 114.135) (end 139.65 122.55) (width 0.25) (layer "B.Cu") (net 1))
 (segment (start 139.65 122.55) (end 139.65 123.9) (width 0.25) (layer "B.Cu") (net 1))
 (segment (start 165.5 114.5) (end 168.7 114.5) (width 0.25) (layer "B.Cu") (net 1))
 (segment (start 180.775 89.425) (end 182.045 90.695) (width 0.25) (layer "B.Cu") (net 1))
 (segment (start 133 113) (end 133.754511 112.245489) (width 0.25) (layer "F.Cu") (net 15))
 (segment (start 133.754511 112.245489) (end 133.754511 98.345489) (width 0.25) (layer "F.Cu") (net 15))
 (segment (start 133.754511 98.345489) (end 136.7 95.4) (width 0.25) (layer "F.Cu") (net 15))
 (segment (start 125.35 116.675) (end 129.325 116.675) (width 0.25) (layer "F.Cu") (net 15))
 (segment (start 129.325 116.675) (end 133 113) (width 0.25) (layer "F.Cu") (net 15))
 (via (at 136.7 95.4) (size 0.8) (drill 0.4) (layers "F.Cu" "B.Cu") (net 15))
 (segment (start 140.07 95.4) (end 145.33 90.14) (width 0.25) (layer "B.Cu") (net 15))
 (segment (start 136.7 95.4) (end 140.07 95.4) (width 0.25) (layer "B.Cu") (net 15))
 (segment (start 137.11 111.59) (end 139 109.7) (width 0.25) (layer "F.Cu") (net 8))
 (segment (start 137.11 123.9) (end 137.11 111.59) (width 0.25) (layer "F.Cu") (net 8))
 (segment (start 139 91.43) (end 137.71 90.14) (width 0.25) (layer "F.Cu") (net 8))
 (segment (start 139 109.7) (end 139 91.43) (width 0.25) (layer "F.Cu") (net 8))
 (segment (start 148 115.67) (end 148 115.8) (width 0.25) (layer "F.Cu") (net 9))
 (segment (start 147.97 115.67) (end 140.7 108.4) (width 0.25) (layer "F.Cu") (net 9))
 (segment (start 148.025 115.825) (end 148.025 124.05) (width 0.25) (layer "F.Cu") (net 9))
 (segment (start 148 115.67) (end 147.97 115.67) (width 0.25) (layer "F.Cu") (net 9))
 (segment (start 148 115.8) (end 148.025 115.825) (width 0.25) (layer "F.Cu") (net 9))
 (via (at 140.7 108.4) (size 0.8) (drill 0.4) (layers "F.Cu" "B.Cu") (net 9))
 (segment (start 140.7 108.37) (end 137.71 105.38) (width 0.25) (layer "B.Cu") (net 9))
 (segment (start 140.7 108.4) (end 140.7 108.37) (width 0.25) (layer "B.Cu") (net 9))
 (segment (start 177.9 108.7) (end 179.505 107.095) (width 0.25) (layer "F.Cu") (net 4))
 (segment (start 151.19 108.7) (end 177.9 108.7) (width 0.25) (layer "F.Cu") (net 4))
 (segment (start 147.87 105.38) (end 151.19 108.7) (width 0.25) (layer "F.Cu") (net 4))
 (segment (start 179.47 123.8) (end 179.47 114.37) (width 0.25) (layer "B.Cu") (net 4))
 (segment (start 180.970489 105.629511) (end 180.970489 104.529511) (width 0.25) (layer "B.Cu") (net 4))
 (segment (start 179.505 107.095) (end 180.970489 105.629511) (width 0.25) (layer "B.Cu") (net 4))
 (segment (start 179.505 107.095) (end 177.205 107.095) (width 0.25) (layer "B.Cu") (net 4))
 (segment (start 178.2 83.04) (end 178.2 73.92) (width 0.25) (layer "B.Cu") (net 4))
 (segment (start 177.205 107.095) (end 175.9 108.4) (width 0.25) (layer "B.Cu") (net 4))
 (segment (start 179.47 114.37) (end 175.9 110.8) (width 0.25) (layer "B.Cu") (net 4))
 (segment (start 185.7 103.7) (end 184.870489 104.529511) (width 0.25) (layer "B.Cu") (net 4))
 (segment (start 178.2 73.92) (end 179.57 72.55) (width 0.25) (layer "B.Cu") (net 4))
 (segment (start 181.910411 87) (end 182.5 87) (width 0.25) (layer "B.Cu") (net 4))
 (segment (start 179.505 84.345) (end 179.505 84.594589) (width 0.25) (layer "B.Cu") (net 4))
 (segment (start 179.505 84.594589) (end 181.910411 87) (width 0.25) (layer "B.Cu") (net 4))
 (segment (start 175.9 108.4) (end 175.9 110.8) (width 0.25) (layer "B.Cu") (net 4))
 (segment (start 185.7 90.2) (end 185.7 103.7) (width 0.25) (layer "B.Cu") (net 4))
 (segment (start 184.870489 104.529511) (end 180.970489 104.529511) (width 0.25) (layer "B.Cu") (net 4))
 (segment (start 179.505 84.345) (end 178.2 83.04) (width 0.25) (layer "B.Cu") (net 4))
 (segment (start 182.5 87) (end 185.7 90.2) (width 0.25) (layer "B.Cu") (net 4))
 (segment (start 181 79.7) (end 181 80.640978) (width 0.25) (layer "F.Cu") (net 3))
 (segment (start 181 80.640978) (end 180.970489 80.670489) (width 0.25) (layer "F.Cu") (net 3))
 (segment (start 152.83 107.8) (end 174.2 107.8) (width 0.25) (layer "F.Cu") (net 3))
 (segment (start 183.4 119.3) (end 181.43 119.3) (width 0.25) (layer "F.Cu") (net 3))
 (segment (start 180.970489 80.670489) (end 180.970489 84.540489) (width 0.25) (layer "F.Cu") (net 3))
 (segment (start 177.824511 78.624511) (end 179.924511 78.624511) (width 0.25) (layer "F.Cu") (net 3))
 (segment (start 181.43 119.3) (end 176.93 123.8) (width 0.25) (layer "F.Cu") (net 3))
 (segment (start 180.970489 84.540489) (end 182.045 85.615) (width 0.25) (layer "F.Cu") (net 3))
 (segment (start 177.03 77.83) (end 177.824511 78.624511) (width 0.25) (layer "F.Cu") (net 3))
 (segment (start 179.924511 78.624511) (end 181 79.7) (width 0.25) (layer "F.Cu") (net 3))
 (segment (start 150.41 105.38) (end 152.83 107.8) (width 0.25) (layer "F.Cu") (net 3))
 (segment (start 177.03 72.55) (end 177.03 77.83) (width 0.25) (layer "F.Cu") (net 3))
 (via (at 174.2 107.8) (size 0.8) (drill 0.4) (layers "F.Cu" "B.Cu") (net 3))
 (via (at 183.4 119.3) (size 0.8) (drill 0.4) (layers "F.Cu" "B.Cu") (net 3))
 (segment (start 183.4 109.72) (end 183.4 119.3) (width 0.25) (layer "B.Cu") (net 3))
 (segment (start 182.045 85.615) (end 186.395479 89.965479) (width 0.25) (layer "B.Cu") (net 3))
 (segment (start 176.93 113.93) (end 174.2 111.2) (width 0.25) (layer "B.Cu") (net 3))
 (segment (start 176.93 123.8) (end 176.93 113.93) (width 0.25) (layer "B.Cu") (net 3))
 (segment (start 182.045 108.365) (end 183.4 109.72) (width 0.25) (layer "B.Cu") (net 3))
 (segment (start 186.395479 104.014521) (end 182.045 108.365) (width 0.25) (layer "B.Cu") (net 3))
 (segment (start 174.2 111.2) (end 174.2 107.8) (width 0.25) (layer "B.Cu") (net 3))
 (segment (start 186.395479 89.965479) (end 186.395479 104.014521) (width 0.25) (layer "B.Cu") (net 3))
 (segment (start 160.68 110.98) (end 160.7 111) (width 0.25) (layer "F.Cu") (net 7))
 (segment (start 153.105 124.05) (end 155.3 121.855) (width 0.25) (layer "F.Cu") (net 7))
 (segment (start 158.03 105.38) (end 158.03 105.6055) (width 0.25) (layer "F.Cu") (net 7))
 (segment (start 155.05 113) (end 157.07 110.98) (width 0.25) (layer "F.Cu") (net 7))
 (segment (start 158.03 105.6055) (end 159.5 107.0755) (width 0.25) (layer "F.Cu") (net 7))
 (segment (start 158.315 110.98) (end 160.68 110.98) (width 0.25) (layer "F.Cu") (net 7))
 (segment (start 157.07 110.98) (end 158.315 110.98) (width 0.25) (layer "F.Cu") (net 7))
 (segment (start 155.3 121.855) (end 155.3 118.5) (width 0.25) (layer "F.Cu") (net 7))
 (via (at 155.3 118.5) (size 0.8) (drill 0.4) (layers "F.Cu" "B.Cu") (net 7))
 (via (at 159.5 107.0755) (size 0.8) (drill 0.4) (layers "F.Cu" "B.Cu") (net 7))
 (via (at 160.7 111) (size 0.8) (drill 0.4) (layers "F.Cu" "B.Cu") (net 7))
 (segment (start 160.7 108.2755) (end 159.5 107.0755) (width 0.25) (layer "B.Cu") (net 7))
 (segment (start 126.405 111.595) (end 126.5 111.5) (width 0.25) (layer "B.Cu") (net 7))
 (segment (start 125.35 111.595) (end 126.405 111.595) (width 0.25) (layer "B.Cu") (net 7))
 (segment (start 126.5 111.5) (end 153.5 111.5) (width 0.25) (layer "B.Cu") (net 7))
 (segment (start 153.5 111.5) (end 155 113) (width 0.25) (layer "B.Cu") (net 7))
 (segment (start 155.1 113.1) (end 155.3 113.3) (width 0.25) (layer "B.Cu") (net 7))
 (segment (start 160.7 111) (end 160.7 108.2755) (width 0.25) (layer "B.Cu") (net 7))
 (segment (start 155 113) (end 155.1 113.1) (width 0.25) (layer "B.Cu") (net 7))
 (segment (start 159.5 107.0755) (end 159.5 108.5) (width 0.25) (layer "B.Cu") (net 7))
 (segment (start 159.5 108.5) (end 155 113) (width 0.25) (layer "B.Cu") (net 7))
 (segment (start 155.3 113.3) (end 155.3 118.5) (width 0.25) (layer "B.Cu") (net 7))
 (segment (start 173.2 114.8) (end 171.4 113) (width 1) (layer "F.Cu") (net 2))
 (segment (start 174.34 114.8) (end 174.3 114.8) (width 1) (layer "F.Cu") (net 2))
 (segment (start 179.505 109.635) (end 176.14 113) (width 1) (layer "F.Cu") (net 2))
 (segment (start 179.505 86.885) (end 180.775 86.885) (width 1) (layer "F.Cu") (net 2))
 (segment (start 162.885 110.98) (end 163.78 110.98) (width 0.25) (layer "F.Cu") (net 2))
 (segment (start 176.14 113) (end 174.34 114.8) (width 1) (layer "F.Cu") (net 2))
 (segment (start 174.3 114.8) (end 173.2 114.8) (width 1) (layer "F.Cu") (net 2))
 (segment (start 184.6 102.5) (end 184.6 108.35) (width 1) (layer "F.Cu") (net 2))
 (segment (start 174.49 72.55) (end 174.49 81.87) (width 1) (layer "F.Cu") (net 2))
 (segment (start 184.6 108.35) (end 182.045 110.905) (width 1) (layer "F.Cu") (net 2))
 (segment (start 174.49 81.87) (end 179.505 86.885) (width 1) (layer "F.Cu") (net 2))
 (segment (start 165.8 113) (end 166.65 113) (width 0.25) (layer "F.Cu") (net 2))
 (segment (start 171.4 113) (end 166.65 113) (width 1) (layer "F.Cu") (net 2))
 (segment (start 163.78 110.98) (end 165.8 113) (width 0.25) (layer "F.Cu") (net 2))
 (segment (start 180.775 86.885) (end 182.045 88.155) (width 1) (layer "F.Cu") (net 2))
 (via (at 174.3 114.8) (size 0.8) (drill 0.4) (layers "F.Cu" "B.Cu") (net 2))
 (via (at 184.6 102.5) (size 0.8) (drill 0.4) (layers "F.Cu" "B.Cu") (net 2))
 (segment (start 135.31 74.69) (end 135.31 74.75) (width 1) (layer "B.Cu") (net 2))
 (segment (start 184.6 90.71) (end 184.6 102.5) (width 1) (layer "B.Cu") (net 2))
 (segment (start 182.045 88.155) (end 184.6 90.71) (width 1) (layer "B.Cu") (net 2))
 (segment (start 139 71) (end 135.31 74.69) (width 1) (layer "B.Cu") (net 2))
 (segment (start 174.3 123.71) (end 174.39 123.8) (width 1) (layer "B.Cu") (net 2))
 (segment (start 173.499022 71) (end 139 71) (width 1) (layer "B.Cu") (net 2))
 (segment (start 182.045 110.905) (end 180.775 110.905) (width 1) (layer "B.Cu") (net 2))
 (segment (start 180.775 110.905) (end 179.505 109.635) (width 1) (layer "B.Cu") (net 2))
 (segment (start 174.3 114.8) (end 174.3 123.71) (width 1) (layer "B.Cu") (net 2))
 (segment (start 174.49 71.990978) (end 173.499022 71) (width 1) (layer "B.Cu") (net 2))
 (segment (start 174.49 72.55) (end 174.49 71.990978) (width 1) (layer "B.Cu") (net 2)))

